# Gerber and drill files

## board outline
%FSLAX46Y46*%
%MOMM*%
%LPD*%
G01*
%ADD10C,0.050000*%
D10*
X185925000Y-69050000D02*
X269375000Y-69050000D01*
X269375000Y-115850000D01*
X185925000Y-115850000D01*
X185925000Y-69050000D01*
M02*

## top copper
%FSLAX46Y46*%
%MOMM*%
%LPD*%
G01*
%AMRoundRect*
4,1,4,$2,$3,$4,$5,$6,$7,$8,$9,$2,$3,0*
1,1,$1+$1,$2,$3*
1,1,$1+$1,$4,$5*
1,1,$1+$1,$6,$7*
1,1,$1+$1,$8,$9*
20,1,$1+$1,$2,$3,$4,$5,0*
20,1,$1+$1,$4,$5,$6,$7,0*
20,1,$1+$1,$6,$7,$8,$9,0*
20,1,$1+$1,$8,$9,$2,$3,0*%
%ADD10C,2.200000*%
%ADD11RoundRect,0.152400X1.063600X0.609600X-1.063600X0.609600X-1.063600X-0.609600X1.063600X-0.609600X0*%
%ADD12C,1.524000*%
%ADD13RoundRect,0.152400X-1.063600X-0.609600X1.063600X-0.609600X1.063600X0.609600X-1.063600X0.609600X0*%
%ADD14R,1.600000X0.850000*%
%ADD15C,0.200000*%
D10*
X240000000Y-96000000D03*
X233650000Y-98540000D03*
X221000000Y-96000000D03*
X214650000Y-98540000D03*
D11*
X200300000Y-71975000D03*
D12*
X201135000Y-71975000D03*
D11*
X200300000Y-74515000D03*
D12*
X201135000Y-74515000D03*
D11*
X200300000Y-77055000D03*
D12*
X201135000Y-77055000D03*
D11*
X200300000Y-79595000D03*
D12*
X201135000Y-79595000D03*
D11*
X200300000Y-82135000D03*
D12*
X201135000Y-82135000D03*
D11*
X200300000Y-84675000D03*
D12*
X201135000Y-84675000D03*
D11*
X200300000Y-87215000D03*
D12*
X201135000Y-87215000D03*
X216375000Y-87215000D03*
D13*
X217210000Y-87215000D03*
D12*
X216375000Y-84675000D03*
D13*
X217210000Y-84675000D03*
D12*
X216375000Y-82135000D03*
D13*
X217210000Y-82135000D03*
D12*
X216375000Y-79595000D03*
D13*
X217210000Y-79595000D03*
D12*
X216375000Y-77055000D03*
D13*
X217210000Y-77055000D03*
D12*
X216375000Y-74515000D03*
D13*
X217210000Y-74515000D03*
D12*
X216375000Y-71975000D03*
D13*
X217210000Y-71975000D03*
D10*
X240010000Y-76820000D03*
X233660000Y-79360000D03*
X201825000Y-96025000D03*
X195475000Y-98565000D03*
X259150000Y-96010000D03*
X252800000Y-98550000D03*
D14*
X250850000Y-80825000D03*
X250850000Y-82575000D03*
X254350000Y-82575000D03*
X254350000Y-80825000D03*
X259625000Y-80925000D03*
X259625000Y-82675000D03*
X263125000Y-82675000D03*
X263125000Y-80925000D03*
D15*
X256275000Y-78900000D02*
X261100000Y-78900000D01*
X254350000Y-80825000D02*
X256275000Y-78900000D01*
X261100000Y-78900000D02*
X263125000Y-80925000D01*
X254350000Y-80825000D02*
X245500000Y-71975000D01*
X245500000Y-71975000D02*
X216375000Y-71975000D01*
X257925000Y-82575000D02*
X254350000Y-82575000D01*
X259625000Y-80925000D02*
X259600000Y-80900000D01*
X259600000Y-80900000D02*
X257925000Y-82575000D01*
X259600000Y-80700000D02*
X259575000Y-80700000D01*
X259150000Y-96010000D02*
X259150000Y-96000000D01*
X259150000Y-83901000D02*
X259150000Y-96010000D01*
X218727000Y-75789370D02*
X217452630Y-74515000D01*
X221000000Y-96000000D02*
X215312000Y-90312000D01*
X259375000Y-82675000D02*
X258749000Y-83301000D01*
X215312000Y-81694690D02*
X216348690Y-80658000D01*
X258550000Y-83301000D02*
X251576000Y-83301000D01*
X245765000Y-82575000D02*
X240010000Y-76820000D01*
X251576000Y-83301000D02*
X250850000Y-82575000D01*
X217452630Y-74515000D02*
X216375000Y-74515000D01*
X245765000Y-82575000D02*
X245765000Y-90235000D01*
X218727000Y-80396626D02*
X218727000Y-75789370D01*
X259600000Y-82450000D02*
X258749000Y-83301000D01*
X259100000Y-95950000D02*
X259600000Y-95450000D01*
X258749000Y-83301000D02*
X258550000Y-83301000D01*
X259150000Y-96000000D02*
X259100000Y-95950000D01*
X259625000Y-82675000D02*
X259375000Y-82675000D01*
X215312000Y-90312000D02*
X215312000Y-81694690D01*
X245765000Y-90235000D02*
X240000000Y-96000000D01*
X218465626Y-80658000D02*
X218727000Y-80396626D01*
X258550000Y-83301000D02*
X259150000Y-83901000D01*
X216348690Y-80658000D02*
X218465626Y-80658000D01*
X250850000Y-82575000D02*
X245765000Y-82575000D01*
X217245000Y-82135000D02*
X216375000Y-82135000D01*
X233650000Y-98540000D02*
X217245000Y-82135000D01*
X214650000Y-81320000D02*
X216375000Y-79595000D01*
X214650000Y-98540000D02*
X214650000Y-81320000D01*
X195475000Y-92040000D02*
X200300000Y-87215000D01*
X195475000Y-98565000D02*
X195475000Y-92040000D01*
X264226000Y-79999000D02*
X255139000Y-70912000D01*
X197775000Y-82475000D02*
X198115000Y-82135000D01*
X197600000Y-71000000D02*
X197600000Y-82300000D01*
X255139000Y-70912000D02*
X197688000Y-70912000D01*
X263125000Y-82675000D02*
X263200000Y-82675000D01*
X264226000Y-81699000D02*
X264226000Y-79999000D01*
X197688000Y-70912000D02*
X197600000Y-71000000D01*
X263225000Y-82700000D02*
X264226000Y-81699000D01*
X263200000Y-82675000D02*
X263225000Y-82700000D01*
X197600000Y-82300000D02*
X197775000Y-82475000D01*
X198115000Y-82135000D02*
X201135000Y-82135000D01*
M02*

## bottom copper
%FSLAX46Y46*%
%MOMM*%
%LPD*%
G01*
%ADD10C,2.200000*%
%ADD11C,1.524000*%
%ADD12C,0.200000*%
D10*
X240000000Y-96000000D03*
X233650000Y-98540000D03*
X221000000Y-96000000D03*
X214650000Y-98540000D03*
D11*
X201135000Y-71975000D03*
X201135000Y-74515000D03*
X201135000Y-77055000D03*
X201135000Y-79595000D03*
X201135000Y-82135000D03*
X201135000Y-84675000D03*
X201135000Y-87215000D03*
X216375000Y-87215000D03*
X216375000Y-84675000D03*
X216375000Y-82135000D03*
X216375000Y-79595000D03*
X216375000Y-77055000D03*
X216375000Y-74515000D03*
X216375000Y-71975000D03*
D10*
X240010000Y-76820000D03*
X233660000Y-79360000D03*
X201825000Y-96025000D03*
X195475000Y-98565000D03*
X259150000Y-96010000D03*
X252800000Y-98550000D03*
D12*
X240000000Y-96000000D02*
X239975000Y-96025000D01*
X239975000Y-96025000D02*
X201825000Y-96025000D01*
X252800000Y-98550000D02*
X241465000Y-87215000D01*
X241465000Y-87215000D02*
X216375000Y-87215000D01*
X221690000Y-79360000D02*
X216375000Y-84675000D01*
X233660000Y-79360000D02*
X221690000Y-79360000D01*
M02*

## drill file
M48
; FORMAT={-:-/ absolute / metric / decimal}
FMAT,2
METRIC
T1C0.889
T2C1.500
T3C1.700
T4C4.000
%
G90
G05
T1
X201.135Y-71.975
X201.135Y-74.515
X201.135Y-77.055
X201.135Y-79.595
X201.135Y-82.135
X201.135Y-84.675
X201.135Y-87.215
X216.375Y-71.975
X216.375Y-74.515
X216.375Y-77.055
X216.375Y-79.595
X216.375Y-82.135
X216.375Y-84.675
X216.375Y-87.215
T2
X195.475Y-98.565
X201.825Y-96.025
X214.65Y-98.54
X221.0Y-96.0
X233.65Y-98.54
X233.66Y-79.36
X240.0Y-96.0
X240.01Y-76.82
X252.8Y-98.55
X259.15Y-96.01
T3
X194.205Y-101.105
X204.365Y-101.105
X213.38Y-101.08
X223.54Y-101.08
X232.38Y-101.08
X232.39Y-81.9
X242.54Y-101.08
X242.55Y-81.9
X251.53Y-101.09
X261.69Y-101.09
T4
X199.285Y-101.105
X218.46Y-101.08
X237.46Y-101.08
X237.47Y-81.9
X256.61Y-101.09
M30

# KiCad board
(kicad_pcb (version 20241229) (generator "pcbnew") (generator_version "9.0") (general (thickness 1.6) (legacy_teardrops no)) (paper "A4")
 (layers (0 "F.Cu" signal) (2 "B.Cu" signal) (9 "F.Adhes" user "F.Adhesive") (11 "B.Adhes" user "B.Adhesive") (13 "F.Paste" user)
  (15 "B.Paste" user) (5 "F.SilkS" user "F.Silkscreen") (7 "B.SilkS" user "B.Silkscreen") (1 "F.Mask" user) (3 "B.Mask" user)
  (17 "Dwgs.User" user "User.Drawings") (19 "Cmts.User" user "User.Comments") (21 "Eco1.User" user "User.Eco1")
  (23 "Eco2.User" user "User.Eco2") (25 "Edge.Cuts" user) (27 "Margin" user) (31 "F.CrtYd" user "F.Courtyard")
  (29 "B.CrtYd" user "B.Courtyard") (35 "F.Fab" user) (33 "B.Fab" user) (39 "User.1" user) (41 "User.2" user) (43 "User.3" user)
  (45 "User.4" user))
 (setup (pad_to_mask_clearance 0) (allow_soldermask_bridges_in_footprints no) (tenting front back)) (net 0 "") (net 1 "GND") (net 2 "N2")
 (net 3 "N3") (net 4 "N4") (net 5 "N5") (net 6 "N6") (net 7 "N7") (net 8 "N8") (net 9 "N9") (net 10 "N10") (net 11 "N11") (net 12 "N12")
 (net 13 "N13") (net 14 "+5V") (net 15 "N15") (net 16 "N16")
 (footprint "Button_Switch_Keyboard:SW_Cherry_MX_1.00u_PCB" (layer "F.Cu") (at 240 96)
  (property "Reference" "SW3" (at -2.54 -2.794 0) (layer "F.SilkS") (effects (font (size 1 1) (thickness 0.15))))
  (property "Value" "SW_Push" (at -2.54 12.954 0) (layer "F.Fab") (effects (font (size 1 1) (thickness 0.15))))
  (pad "" np_thru_hole circle (at -7.62 5.08) (size 1.7 1.7) (drill 1.7) (layers "*.Cu" "*.Mask"))
  (pad "" np_thru_hole circle (at -2.54 5.08) (size 4 4) (drill 4) (layers "*.Cu" "*.Mask"))
  (pad "" np_thru_hole circle (at 2.54 5.08) (size 1.7 1.7) (drill 1.7) (layers "*.Cu" "*.Mask"))
  (pad "1" thru_hole circle (at 0 0) (size 2.2 2.2) (drill 1.5) (layers "*.Cu" "*.Mask") (remove_unused_layers no) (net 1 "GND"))
  (pad "2" thru_hole circle (at -6.35 2.54) (size 2.2 2.2) (drill 1.5) (layers "*.Cu" "*.Mask") (remove_unused_layers no) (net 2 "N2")))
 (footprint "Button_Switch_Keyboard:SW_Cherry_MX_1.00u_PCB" (layer "F.Cu") (at 221 96)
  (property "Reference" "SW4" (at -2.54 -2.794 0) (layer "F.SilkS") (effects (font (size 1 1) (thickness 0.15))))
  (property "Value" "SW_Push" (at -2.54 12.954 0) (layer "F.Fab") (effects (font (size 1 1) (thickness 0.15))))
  (pad "" np_thru_hole circle (at -7.62 5.08) (size 1.7 1.7) (drill 1.7) (layers "*.Cu" "*.Mask"))
  (pad "" np_thru_hole circle (at -2.54 5.08) (size 4 4) (drill 4) (layers "*.Cu" "*.Mask"))
  (pad "" np_thru_hole circle (at 2.54 5.08) (size 1.7 1.7) (drill 1.7) (layers "*.Cu" "*.Mask"))
  (pad "1" thru_hole circle (at 0 0) (size 2.2 2.2) (drill 1.5) (layers "*.Cu" "*.Mask") (remove_unused_layers no) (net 1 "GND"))
  (pad "2" thru_hole circle (at -6.35 2.54) (size 2.2 2.2) (drill 1.5) (layers "*.Cu" "*.Mask") (remove_unused_layers no) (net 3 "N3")))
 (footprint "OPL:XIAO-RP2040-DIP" (layer "F.Cu") (at 208.755 79.595)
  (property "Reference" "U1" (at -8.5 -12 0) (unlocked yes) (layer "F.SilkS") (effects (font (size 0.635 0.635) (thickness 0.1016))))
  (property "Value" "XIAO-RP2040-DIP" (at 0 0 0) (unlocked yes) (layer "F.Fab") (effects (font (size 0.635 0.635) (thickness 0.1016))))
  (pad "1" smd roundrect (at -8.455 -7.62 180) (size 2.432 1.524) (layers "F.Cu" "F.Mask") (roundrect_rratio 0.1) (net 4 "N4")
   (thermal_bridge_angle 45))
  (pad "1" thru_hole circle (at -7.62 -7.62 180) (size 1.524 1.524) (drill 0.889) (layers "*.Cu" "*.Mask") (remove_unused_layers no)
   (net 4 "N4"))
  (pad "2" smd roundrect (at -8.455 -5.08 180) (size 2.432 1.524) (layers "F.Cu" "F.Mask") (roundrect_rratio 0.1) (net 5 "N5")
   (thermal_bridge_angle 45))
  (pad "2" thru_hole circle (at -7.62 -5.08 180) (size 1.524 1.524) (drill 0.889) (layers "*.Cu" "*.Mask") (remove_unused_layers no)
   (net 5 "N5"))
  (pad "3" smd roundrect (at -8.455 -2.54 180) (size 2.432 1.524) (layers "F.Cu" "F.Mask") (roundrect_rratio 0.1) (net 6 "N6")
   (thermal_bridge_angle 45))
  (pad "3" thru_hole circle (at -7.62 -2.54 180) (size 1.524 1.524) (drill 0.889) (layers "*.Cu" "*.Mask") (remove_unused_layers no)
   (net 6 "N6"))
  (pad "4" smd roundrect (at -8.455 0 180) (size 2.432 1.524) (layers "F.Cu" "F.Mask") (roundrect_rratio 0.1) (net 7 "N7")
   (thermal_bridge_angle 45))
  (pad "4" thru_hole circle (at -7.62 0 180) (size 1.524 1.524) (drill 0.889) (layers "*.Cu" "*.Mask") (remove_unused_layers no)
   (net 7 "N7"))
  (pad "5" smd roundrect (at -8.455 2.54 180) (size 2.432 1.524) (layers "F.Cu" "F.Mask") (roundrect_rratio 0.1) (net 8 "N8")
   (thermal_bridge_angle 45))
  (pad "5" thru_hole circle (at -7.62 2.54 180) (size 1.524 1.524) (drill 0.889) (layers "*.Cu" "*.Mask") (remove_unused_layers no)
   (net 8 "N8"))
  (pad "6" smd roundrect (at -8.455 5.08 180) (size 2.432 1.524) (layers "F.Cu" "F.Mask") (roundrect_rratio 0.1) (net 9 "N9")
   (thermal_bridge_angle 45))
  (pad "6" thru_hole circle (at -7.62 5.08 180) (size 1.524 1.524) (drill 0.889) (layers "*.Cu" "*.Mask") (remove_unused_layers no)
   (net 9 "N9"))
  (pad "7" smd roundrect (at -8.455 7.62 180) (size 2.432 1.524) (layers "F.Cu" "F.Mask") (roundrect_rratio 0.1) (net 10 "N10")
   (thermal_bridge_angle 45))
  (pad "7" thru_hole circle (at -7.62 7.62 180) (size 1.524 1.524) (drill 0.889) (layers "*.Cu" "*.Mask") (remove_unused_layers no)
   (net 10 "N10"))
  (pad "8" thru_hole circle (at 7.62 7.62) (size 1.524 1.524) (drill 0.889) (layers "*.Cu" "*.Mask") (remove_unused_layers no)
   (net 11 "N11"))
  (pad "8" smd roundrect (at 8.455 7.62) (size 2.432 1.524) (layers "F.Cu" "F.Mask") (roundrect_rratio 0.1) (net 11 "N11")
   (thermal_bridge_angle 45))
  (pad "9" thru_hole circle (at 7.62 5.08) (size 1.524 1.524) (drill 0.889) (layers "*.Cu" "*.Mask") (remove_unused_layers no)
   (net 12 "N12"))
  (pad "9" smd roundrect (at 8.455 5.08) (size 2.432 1.524) (layers "F.Cu" "F.Mask") (roundrect_rratio 0.1) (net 12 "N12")
   (thermal_bridge_angle 45))
  (pad "10" thru_hole circle (at 7.62 2.54) (size 1.524 1.524) (drill 0.889) (layers "*.Cu" "*.Mask") (remove_unused_layers no) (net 2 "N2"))
  (pad "10" smd roundrect (at 8.455 2.54) (size 2.432 1.524) (layers "F.Cu" "F.Mask") (roundrect_rratio 0.1) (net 2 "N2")
   (thermal_bridge_angle 45))
  (pad "11" thru_hole circle (at 7.62 0) (size 1.524 1.524) (drill 0.889) (layers "*.Cu" "*.Mask") (remove_unused_layers no) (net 3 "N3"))
  (pad "11" smd roundrect (at 8.455 0) (size 2.432 1.524) (layers "F.Cu" "F.Mask") (roundrect_rratio 0.1) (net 3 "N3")
   (thermal_bridge_angle 45))
  (pad "12" thru_hole circle (at 7.62 -2.54) (size 1.524 1.524) (drill 0.889) (layers "*.Cu" "*.Mask") (remove_unused_layers no)
   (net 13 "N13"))
  (pad "12" smd roundrect (at 8.455 -2.54) (size 2.432 1.524) (layers "F.Cu" "F.Mask") (roundrect_rratio 0.1) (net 13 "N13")
   (thermal_bridge_angle 45))
  (pad "13" thru_hole circle (at 7.62 -5.08) (size 1.524 1.524) (drill 0.889) (layers "*.Cu" "*.Mask") (remove_unused_layers no)
   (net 1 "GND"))
  (pad "13" smd roundrect (at 8.455 -5.08) (size 2.432 1.524) (layers "F.Cu" "F.Mask") (roundrect_rratio 0.1) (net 1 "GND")
   (thermal_bridge_angle 45))
  (pad "14" thru_hole circle (at 7.62 -7.62) (size 1.524 1.524) (drill 0.889) (layers "*.Cu" "*.Mask") (remove_unused_layers no)
   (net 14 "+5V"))
  (pad "14" smd roundrect (at 8.455 -7.62) (size 2.432 1.524) (layers "F.Cu" "F.Mask") (roundrect_rratio 0.1) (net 14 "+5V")
   (thermal_bridge_angle 45)))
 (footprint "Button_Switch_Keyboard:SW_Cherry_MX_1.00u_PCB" (layer "F.Cu") (at 240.01 76.82)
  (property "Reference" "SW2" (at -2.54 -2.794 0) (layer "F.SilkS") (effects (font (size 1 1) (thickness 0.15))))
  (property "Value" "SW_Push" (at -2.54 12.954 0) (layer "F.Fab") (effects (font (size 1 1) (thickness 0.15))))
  (pad "" np_thru_hole circle (at -7.62 5.08) (size 1.7 1.7) (drill 1.7) (layers "*.Cu" "*.Mask"))
  (pad "" np_thru_hole circle (at -2.54 5.08) (size 4 4) (drill 4) (layers "*.Cu" "*.Mask"))
  (pad "" np_thru_hole circle (at 2.54 5.08) (size 1.7 1.7) (drill 1.7) (layers "*.Cu" "*.Mask"))
  (pad "1" thru_hole circle (at 0 0) (size 2.2 2.2) (drill 1.5) (layers "*.Cu" "*.Mask") (remove_unused_layers no) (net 1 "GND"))
  (pad "2" thru_hole circle (at -6.35 2.54) (size 2.2 2.2) (drill 1.5) (layers "*.Cu" "*.Mask") (remove_unused_layers no) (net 12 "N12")))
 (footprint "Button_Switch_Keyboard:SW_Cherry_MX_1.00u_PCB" (layer "F.Cu") (at 201.825 96.025)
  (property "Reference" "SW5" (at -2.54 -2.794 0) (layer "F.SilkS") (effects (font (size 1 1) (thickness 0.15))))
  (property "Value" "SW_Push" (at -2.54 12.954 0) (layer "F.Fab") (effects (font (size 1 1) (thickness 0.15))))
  (pad "" np_thru_hole circle (at -7.62 5.08) (size 1.7 1.7) (drill 1.7) (layers "*.Cu" "*.Mask"))
  (pad "" np_thru_hole circle (at -2.54 5.08) (size 4 4) (drill 4) (layers "*.Cu" "*.Mask"))
  (pad "" np_thru_hole circle (at 2.54 5.08) (size 1.7 1.7) (drill 1.7) (layers "*.Cu" "*.Mask"))
  (pad "1" thru_hole circle (at 0 0) (size 2.2 2.2) (drill 1.5) (layers "*.Cu" "*.Mask") (remove_unused_layers no) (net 1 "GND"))
  (pad "2" thru_hole circle (at -6.35 2.54) (size 2.2 2.2) (drill 1.5) (layers "*.Cu" "*.Mask") (remove_unused_layers no) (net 10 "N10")))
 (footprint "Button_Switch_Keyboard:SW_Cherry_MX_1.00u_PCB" (layer "F.Cu") (at 259.15 96.01)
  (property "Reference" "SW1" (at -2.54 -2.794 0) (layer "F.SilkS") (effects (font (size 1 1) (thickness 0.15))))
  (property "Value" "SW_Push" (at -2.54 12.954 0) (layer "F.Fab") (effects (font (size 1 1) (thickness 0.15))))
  (pad "" np_thru_hole circle (at -7.62 5.08) (size 1.7 1.7) (drill 1.7) (layers "*.Cu" "*.Mask"))
  (pad "" np_thru_hole circle (at -2.54 5.08) (size 4 4) (drill 4) (layers "*.Cu" "*.Mask"))
  (pad "" np_thru_hole circle (at 2.54 5.08) (size 1.7 1.7) (drill 1.7) (layers "*.Cu" "*.Mask"))
  (pad "1" thru_hole circle (at 0 0) (size 2.2 2.2) (drill 1.5) (layers "*.Cu" "*.Mask") (remove_unused_layers no) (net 1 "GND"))
  (pad "2" thru_hole circle (at -6.35 2.54) (size 2.2 2.2) (drill 1.5) (layers "*.Cu" "*.Mask") (remove_unused_layers no) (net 11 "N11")))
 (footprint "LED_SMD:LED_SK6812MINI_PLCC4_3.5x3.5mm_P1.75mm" (layer "F.Cu") (at 252.6 81.7)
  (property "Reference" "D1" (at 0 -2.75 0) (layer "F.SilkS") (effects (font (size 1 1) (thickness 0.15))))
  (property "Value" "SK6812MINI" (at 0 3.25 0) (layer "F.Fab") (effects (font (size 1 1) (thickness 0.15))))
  (pad "1" smd rect (at -1.75 -0.875) (size 1.6 0.85) (layers "F.Cu" "F.Mask" "F.Paste") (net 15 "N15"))
  (pad "2" smd rect (at -1.75 0.875) (size 1.6 0.85) (layers "F.Cu" "F.Mask" "F.Paste") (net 1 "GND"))
  (pad "3" smd rect (at 1.75 0.875) (size 1.6 0.85) (layers "F.Cu" "F.Mask" "F.Paste") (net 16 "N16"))
  (pad "4" smd rect (at 1.75 -0.875) (size 1.6 0.85) (layers "F.Cu" "F.Mask" "F.Paste") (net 14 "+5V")))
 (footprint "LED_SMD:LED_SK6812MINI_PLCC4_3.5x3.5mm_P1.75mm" (layer "F.Cu") (at 261.375 81.8)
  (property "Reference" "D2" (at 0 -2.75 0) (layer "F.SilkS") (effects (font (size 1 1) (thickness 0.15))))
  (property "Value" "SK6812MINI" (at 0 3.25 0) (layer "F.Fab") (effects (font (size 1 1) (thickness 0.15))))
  (pad "1" smd rect (at -1.75 -0.875) (size 1.6 0.85) (layers "F.Cu" "F.Mask" "F.Paste") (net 16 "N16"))
  (pad "2" smd rect (at -1.75 0.875) (size 1.6 0.85) (layers "F.Cu" "F.Mask" "F.Paste") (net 1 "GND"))
  (pad "3" smd rect (at 1.75 0.875) (size 1.6 0.85) (layers "F.Cu" "F.Mask" "F.Paste") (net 8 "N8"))
  (pad "4" smd rect (at 1.75 -0.875) (size 1.6 0.85) (layers "F.Cu" "F.Mask" "F.Paste") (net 14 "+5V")))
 (gr_rect (start 185.925 69.05) (end 269.375 115.85) (stroke (width 0.05) (type default)) (fill no) (layer "Edge.Cuts"))
 (segment (start 256.275 78.9) (end 261.1 78.9) (width 0.2) (layer "F.Cu") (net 14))
 (segment (start 254.35 80.825) (end 256.275 78.9) (width 0.2) (layer "F.Cu") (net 14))
 (segment (start 261.1 78.9) (end 263.125 80.925) (width 0.2) (layer "F.Cu") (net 14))
 (segment (start 254.35 80.825) (end 245.5 71.975) (width 0.2) (layer "F.Cu") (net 14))
 (segment (start 245.5 71.975) (end 216.375 71.975) (width 0.2) (layer "F.Cu") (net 14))
 (segment (start 257.925 82.575) (end 254.35 82.575) (width 0.2) (layer "F.Cu") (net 16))
 (segment (start 259.625 80.925) (end 259.6 80.9) (width 0.2) (layer "F.Cu") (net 16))
 (segment (start 259.6 80.9) (end 257.925 82.575) (width 0.2) (layer "F.Cu") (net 16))
 (segment (start 259.6 80.7) (end 259.575 80.7) (width 0.2) (layer "F.Cu") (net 16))
 (segment (start 259.15 96.01) (end 259.15 96) (width 0.2) (layer "F.Cu") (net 1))
 (segment (start 259.15 83.901) (end 259.15 96.01) (width 0.2) (layer "F.Cu") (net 1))
 (segment (start 218.727 75.78937) (end 217.45263 74.515) (width 0.2) (layer "F.Cu") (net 1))
 (segment (start 221 96) (end 215.312 90.312) (width 0.2) (layer "F.Cu") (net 1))
 (segment (start 259.375 82.675) (end 258.749 83.301) (width 0.2) (layer "F.Cu") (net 1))
 (segment (start 215.312 81.69469) (end 216.34869 80.658) (width 0.2) (layer "F.Cu") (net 1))
 (segment (start 258.55 83.301) (end 251.576 83.301) (width 0.2) (layer "F.Cu") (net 1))
 (segment (start 245.765 82.575) (end 240.01 76.82) (width 0.2) (layer "F.Cu") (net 1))
 (segment (start 251.576 83.301) (end 250.85 82.575) (width 0.2) (layer "F.Cu") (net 1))
 (segment (start 217.45263 74.515) (end 216.375 74.515) (width 0.2) (layer "F.Cu") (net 1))
 (segment (start 245.765 82.575) (end 245.765 90.235) (width 0.2) (layer "F.Cu") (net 1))
 (segment (start 218.727 80.396626) (end 218.727 75.78937) (width 0.2) (layer "F.Cu") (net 1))
 (segment (start 259.6 82.45) (end 258.749 83.301) (width 0.2) (layer "F.Cu") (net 1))
 (segment (start 259.1 95.95) (end 259.6 95.45) (width 0.2) (layer "F.Cu") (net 1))
 (segment (start 258.749 83.301) (end 258.55 83.301) (width 0.2) (layer "F.Cu") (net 1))
 (segment (start 259.15 96) (end 259.1 95.95) (width 0.2) (layer "F.Cu") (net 1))
 (segment (start 259.625 82.675) (end 259.375 82.675) (width 0.2) (layer "F.Cu") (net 1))
 (segment (start 215.312 90.312) (end 215.312 81.69469) (width 0.2) (layer "F.Cu") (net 1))
 (segment (start 245.765 90.235) (end 240 96) (width 0.2) (layer "F.Cu") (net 1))
 (segment (start 218.465626 80.658) (end 218.727 80.396626) (width 0.2) (layer "F.Cu") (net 1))
 (segment (start 258.55 83.301) (end 259.15 83.901) (width 0.2) (layer "F.Cu") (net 1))
 (segment (start 216.34869 80.658) (end 218.465626 80.658) (width 0.2) (layer "F.Cu") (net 1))
 (segment (start 250.85 82.575) (end 245.765 82.575) (width 0.2) (layer "F.Cu") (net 1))
 (segment (start 240 96) (end 239.975 96.025) (width 0.2) (layer "B.Cu") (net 1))
 (segment (start 239.975 96.025) (end 201.825 96.025) (width 0.2) (layer "B.Cu") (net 1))
 (segment (start 252.8 98.55) (end 241.465 87.215) (width 0.2) (layer "B.Cu") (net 11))
 (segment (start 241.465 87.215) (end 216.375 87.215) (width 0.2) (layer "B.Cu") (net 11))
 (segment (start 221.69 79.36) (end 216.375 84.675) (width 0.2) (layer "B.Cu") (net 12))
 (segment (start 233.66 79.36) (end 221.69 79.36) (width 0.2) (layer "B.Cu") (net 12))
 (segment (start 217.245 82.135) (end 216.375 82.135) (width 0.2) (layer "F.Cu") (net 2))
 (segment (start 233.65 98.54) (end 217.245 82.135) (width 0.2) (layer "F.Cu") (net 2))
 (segment (start 214.65 81.32) (end 216.375 79.595) (width 0.2) (layer "F.Cu") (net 3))
 (segment (start 214.65 98.54) (end 214.65 81.32) (width 0.2) (layer "F.Cu") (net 3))
 (segment (start 195.475 92.04) (end 200.3 87.215) (width 0.2) (layer "F.Cu") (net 10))
 (segment (start 195.475 98.565) (end 195.475 92.04) (width 0.2) (layer "F.Cu") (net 10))
 (segment (start 264.226 79.999) (end 255.139 70.912) (width 0.2) (layer "F.Cu") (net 8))
 (segment (start 197.775 82.475) (end 198.115 82.135) (width 0.2) (layer "F.Cu") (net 8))
 (segment (start 197.6 71) (end 197.6 82.3) (width 0.2) (layer "F.Cu") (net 8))
 (segment (start 255.139 70.912) (end 197.688 70.912) (width 0.2) (layer "F.Cu") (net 8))
 (segment (start 263.125 82.675) (end 263.2 82.675) (width 0.2) (layer "F.Cu") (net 8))
 (segment (start 264.226 81.699) (end 264.226 79.999) (width 0.2) (layer "F.Cu") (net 8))
 (segment (start 197.688 70.912) (end 197.6 71) (width 0.2) (layer "F.Cu") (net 8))
 (segment (start 263.225 82.7) (end 264.226 81.699) (width 0.2) (layer "F.Cu") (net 8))
 (segment (start 263.2 82.675) (end 263.225 82.7) (width 0.2) (layer "F.Cu") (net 8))
 (segment (start 197.6 82.3) (end 197.775 82.475) (width 0.2) (layer "F.Cu") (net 8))
 (segment (start 198.115 82.135) (end 201.135 82.135) (width 0.2) (layer "F.Cu") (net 8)))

